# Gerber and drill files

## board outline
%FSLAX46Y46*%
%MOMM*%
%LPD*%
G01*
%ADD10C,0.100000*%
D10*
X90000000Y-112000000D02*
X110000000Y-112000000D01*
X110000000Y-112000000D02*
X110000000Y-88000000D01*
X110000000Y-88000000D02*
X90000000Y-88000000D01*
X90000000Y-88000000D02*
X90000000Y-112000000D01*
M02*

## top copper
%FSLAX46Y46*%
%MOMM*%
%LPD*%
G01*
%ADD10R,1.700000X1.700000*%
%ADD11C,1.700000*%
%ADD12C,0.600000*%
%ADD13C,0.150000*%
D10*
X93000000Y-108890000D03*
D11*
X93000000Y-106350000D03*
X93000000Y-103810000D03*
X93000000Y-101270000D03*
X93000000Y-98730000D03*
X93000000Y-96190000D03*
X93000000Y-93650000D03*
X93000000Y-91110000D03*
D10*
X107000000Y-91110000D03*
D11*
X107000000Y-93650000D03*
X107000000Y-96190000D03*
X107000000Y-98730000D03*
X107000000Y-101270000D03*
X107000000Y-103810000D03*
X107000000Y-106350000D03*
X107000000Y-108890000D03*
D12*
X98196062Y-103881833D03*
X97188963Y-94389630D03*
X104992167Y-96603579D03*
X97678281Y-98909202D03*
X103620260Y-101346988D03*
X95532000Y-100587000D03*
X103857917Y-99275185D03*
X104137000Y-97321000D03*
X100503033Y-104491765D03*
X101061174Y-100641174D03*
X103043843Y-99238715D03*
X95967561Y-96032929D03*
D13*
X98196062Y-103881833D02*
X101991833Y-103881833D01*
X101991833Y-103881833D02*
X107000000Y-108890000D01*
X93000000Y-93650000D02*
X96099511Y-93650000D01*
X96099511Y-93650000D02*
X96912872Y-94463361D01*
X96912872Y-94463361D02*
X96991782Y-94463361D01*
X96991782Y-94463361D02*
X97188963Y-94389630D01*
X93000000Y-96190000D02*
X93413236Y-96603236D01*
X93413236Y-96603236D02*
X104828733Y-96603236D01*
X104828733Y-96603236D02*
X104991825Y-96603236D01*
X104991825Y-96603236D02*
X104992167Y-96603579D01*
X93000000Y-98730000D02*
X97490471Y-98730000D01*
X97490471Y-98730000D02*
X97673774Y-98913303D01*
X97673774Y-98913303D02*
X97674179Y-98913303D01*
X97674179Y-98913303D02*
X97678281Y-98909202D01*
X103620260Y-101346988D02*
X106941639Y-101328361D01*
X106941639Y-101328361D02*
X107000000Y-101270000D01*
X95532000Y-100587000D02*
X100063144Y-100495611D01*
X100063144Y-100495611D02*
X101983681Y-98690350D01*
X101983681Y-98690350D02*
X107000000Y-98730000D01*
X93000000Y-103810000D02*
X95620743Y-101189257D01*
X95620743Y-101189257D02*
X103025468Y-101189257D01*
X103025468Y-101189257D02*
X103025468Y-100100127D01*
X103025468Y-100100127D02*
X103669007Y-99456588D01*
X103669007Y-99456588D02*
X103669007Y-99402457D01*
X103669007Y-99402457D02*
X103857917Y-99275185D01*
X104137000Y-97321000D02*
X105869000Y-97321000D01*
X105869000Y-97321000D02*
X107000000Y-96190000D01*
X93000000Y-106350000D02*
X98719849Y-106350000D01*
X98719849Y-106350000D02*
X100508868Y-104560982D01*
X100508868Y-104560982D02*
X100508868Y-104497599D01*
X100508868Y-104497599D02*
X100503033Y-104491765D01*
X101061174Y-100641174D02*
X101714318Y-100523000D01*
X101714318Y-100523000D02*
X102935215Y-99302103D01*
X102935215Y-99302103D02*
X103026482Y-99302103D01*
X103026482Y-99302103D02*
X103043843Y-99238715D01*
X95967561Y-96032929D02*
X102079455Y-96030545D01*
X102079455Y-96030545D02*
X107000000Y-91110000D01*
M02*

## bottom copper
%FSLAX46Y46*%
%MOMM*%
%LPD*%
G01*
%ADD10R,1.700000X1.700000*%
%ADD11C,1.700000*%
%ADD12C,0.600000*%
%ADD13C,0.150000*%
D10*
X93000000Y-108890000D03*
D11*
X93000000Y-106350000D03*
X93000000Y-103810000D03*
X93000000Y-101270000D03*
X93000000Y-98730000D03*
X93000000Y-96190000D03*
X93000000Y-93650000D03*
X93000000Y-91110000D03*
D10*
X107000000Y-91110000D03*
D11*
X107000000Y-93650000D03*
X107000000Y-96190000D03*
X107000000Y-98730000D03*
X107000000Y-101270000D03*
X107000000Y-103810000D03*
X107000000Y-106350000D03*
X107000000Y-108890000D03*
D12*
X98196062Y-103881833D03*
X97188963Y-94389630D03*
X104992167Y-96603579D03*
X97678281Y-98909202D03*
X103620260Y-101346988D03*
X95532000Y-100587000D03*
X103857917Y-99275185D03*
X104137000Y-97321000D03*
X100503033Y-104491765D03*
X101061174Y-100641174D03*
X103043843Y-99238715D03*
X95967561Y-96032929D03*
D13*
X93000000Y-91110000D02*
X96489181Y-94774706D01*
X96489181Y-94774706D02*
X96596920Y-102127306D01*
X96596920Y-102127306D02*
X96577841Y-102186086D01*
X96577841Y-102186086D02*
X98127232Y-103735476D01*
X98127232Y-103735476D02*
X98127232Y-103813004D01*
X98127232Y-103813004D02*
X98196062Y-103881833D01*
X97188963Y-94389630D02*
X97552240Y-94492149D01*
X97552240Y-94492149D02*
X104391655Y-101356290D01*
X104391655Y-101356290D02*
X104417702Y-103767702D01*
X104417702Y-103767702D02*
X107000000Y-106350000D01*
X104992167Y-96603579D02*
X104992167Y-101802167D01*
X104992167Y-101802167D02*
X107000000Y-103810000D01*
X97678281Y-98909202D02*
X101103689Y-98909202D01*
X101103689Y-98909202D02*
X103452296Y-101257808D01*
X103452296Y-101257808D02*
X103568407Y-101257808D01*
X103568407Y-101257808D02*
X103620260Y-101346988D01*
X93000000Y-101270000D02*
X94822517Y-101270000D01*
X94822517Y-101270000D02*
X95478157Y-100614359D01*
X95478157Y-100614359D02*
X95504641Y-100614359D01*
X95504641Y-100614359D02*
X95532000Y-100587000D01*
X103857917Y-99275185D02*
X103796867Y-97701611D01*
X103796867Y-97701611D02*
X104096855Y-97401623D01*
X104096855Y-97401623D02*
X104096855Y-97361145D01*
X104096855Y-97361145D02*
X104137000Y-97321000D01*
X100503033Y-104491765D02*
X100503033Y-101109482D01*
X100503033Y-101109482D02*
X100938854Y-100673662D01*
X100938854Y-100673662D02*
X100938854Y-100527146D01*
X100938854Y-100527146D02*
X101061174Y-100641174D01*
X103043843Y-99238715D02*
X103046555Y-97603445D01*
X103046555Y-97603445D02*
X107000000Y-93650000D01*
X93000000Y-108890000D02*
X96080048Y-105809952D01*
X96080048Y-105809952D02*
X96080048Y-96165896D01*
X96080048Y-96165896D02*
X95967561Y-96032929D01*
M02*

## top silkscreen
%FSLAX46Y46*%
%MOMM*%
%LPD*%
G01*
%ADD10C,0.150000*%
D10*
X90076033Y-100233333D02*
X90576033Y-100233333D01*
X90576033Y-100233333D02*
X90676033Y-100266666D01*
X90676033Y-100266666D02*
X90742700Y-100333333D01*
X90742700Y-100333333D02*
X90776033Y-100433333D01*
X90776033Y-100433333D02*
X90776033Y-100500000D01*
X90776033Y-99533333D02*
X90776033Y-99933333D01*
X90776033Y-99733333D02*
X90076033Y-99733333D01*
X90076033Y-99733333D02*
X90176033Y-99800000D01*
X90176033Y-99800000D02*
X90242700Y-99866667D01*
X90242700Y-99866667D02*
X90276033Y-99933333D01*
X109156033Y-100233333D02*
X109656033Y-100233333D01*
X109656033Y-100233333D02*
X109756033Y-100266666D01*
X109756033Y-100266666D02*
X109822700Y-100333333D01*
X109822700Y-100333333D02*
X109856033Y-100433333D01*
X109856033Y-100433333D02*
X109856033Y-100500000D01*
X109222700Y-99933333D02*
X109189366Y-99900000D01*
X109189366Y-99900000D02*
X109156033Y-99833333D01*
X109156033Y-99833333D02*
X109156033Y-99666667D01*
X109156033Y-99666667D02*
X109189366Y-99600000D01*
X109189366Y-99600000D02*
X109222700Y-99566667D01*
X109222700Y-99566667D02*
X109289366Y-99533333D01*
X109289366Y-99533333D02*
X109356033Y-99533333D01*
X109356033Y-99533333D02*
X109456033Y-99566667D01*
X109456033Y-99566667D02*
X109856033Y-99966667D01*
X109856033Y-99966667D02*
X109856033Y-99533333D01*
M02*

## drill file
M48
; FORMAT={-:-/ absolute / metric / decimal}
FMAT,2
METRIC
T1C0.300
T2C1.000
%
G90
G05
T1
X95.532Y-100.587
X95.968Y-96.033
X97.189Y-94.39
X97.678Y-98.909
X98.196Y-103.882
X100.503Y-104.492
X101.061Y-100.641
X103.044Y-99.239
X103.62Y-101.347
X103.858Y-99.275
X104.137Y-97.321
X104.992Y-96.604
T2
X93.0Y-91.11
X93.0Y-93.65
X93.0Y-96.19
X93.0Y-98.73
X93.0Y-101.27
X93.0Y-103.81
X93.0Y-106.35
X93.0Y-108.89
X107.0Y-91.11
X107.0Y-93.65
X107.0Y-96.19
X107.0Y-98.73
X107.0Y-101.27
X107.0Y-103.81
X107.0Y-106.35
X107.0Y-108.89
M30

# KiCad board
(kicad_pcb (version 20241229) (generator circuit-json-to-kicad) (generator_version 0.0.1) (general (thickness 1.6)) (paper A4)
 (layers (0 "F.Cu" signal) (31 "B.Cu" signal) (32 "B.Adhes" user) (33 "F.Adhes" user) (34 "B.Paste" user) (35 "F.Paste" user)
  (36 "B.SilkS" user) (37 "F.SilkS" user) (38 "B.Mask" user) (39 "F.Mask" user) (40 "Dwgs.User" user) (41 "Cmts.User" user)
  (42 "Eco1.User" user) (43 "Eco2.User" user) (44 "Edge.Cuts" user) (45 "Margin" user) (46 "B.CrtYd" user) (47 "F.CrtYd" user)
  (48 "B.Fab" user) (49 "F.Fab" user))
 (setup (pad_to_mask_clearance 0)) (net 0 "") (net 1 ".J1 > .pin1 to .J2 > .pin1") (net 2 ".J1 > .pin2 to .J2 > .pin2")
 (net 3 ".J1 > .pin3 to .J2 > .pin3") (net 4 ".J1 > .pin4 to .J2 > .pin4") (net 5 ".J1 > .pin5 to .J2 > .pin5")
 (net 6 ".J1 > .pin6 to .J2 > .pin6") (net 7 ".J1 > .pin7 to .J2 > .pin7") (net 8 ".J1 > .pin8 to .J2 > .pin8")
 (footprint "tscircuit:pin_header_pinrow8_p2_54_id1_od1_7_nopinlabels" (layer F.Cu) (at 93 100 90)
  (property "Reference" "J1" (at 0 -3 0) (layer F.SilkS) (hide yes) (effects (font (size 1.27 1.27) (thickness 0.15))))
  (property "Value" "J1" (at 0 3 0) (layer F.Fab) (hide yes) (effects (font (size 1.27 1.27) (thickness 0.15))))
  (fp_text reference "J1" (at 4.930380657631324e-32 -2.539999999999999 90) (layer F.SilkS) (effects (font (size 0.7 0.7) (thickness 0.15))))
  (pad "1" thru_hole rect (at -8.89 -3.4382291747912674e-16 90) (size 1.7 1.7) (drill 1) (layers *.Cu *.Mask)
   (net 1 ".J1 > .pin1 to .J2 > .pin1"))
  (pad "2" thru_hole circle (at -6.3500000000000005 3.8882535872928466e-16 0) (size 1.7 1.7) (drill 1) (layers *.Cu *.Mask)
   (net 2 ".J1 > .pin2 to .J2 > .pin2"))
  (pad "3" thru_hole circle (at -3.8100000000000005 2.332952152375708e-16 0) (size 1.7 1.7) (drill 1) (layers *.Cu *.Mask)
   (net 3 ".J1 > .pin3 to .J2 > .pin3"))
  (pad "4" thru_hole circle (at -1.2700000000000005 7.776507174585695e-17 0) (size 1.7 1.7) (drill 1) (layers *.Cu *.Mask)
   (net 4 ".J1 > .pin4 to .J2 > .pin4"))
  (pad "5" thru_hole circle (at 1.2699999999999996 -7.77650717458569e-17 0) (size 1.7 1.7) (drill 1) (layers *.Cu *.Mask)
   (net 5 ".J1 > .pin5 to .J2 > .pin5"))
  (pad "6" thru_hole circle (at 3.8099999999999987 -2.3329521523757073e-16 0) (size 1.7 1.7) (drill 1) (layers *.Cu *.Mask)
   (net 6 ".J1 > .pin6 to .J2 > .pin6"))
  (pad "7" thru_hole circle (at 6.35 -3.888253587292846e-16 0) (size 1.7 1.7) (drill 1) (layers *.Cu *.Mask)
   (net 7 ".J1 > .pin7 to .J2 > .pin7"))
  (pad "8" thru_hole circle (at 8.89 3.4382291747912674e-16 0) (size 1.7 1.7) (drill 1) (layers *.Cu *.Mask)
   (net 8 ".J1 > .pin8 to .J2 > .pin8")))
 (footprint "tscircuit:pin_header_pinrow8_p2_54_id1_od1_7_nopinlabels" (layer F.Cu) (at 107 100 270)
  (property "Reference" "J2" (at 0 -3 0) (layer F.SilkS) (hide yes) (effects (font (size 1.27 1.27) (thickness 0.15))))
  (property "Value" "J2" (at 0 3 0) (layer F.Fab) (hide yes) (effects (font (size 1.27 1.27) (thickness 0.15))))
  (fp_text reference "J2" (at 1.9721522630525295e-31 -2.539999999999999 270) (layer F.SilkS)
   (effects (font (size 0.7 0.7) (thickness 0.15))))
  (pad "1" thru_hole rect (at -8.89 -1.43290332737255e-16 270) (size 1.7 1.7) (drill 1) (layers *.Cu *.Mask)
   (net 1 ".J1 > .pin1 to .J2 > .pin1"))
  (pad "2" thru_hole circle (at -6.3500000000000005 2.782976564877288e-16 0) (size 1.7 1.7) (drill 1) (layers *.Cu *.Mask)
   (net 2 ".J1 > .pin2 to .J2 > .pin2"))
  (pad "3" thru_hole circle (at -3.8100000000000005 -1.8829277398741286e-16 0) (size 1.7 1.7) (drill 1) (layers *.Cu *.Mask)
   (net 3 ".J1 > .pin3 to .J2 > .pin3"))
  (pad "4" thru_hole circle (at -1.2700000000000005 2.3329521523757087e-16 0) (size 1.7 1.7) (drill 1) (layers *.Cu *.Mask)
   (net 4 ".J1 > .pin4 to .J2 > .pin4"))
  (pad "5" thru_hole circle (at 1.2699999999999996 -2.332952152375707e-16 0) (size 1.7 1.7) (drill 1) (layers *.Cu *.Mask)
   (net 5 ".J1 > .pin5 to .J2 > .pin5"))
  (pad "6" thru_hole circle (at 3.8099999999999987 1.8829277398741315e-16 0) (size 1.7 1.7) (drill 1) (layers *.Cu *.Mask)
   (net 6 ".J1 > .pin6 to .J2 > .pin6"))
  (pad "7" thru_hole circle (at 6.35 -2.782976564877286e-16 0) (size 1.7 1.7) (drill 1) (layers *.Cu *.Mask)
   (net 7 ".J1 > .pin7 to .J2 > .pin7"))
  (pad "8" thru_hole circle (at 8.89 1.43290332737255e-16 0) (size 1.7 1.7) (drill 1) (layers *.Cu *.Mask)
   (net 8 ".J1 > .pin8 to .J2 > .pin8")))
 (segment (start 93 91.11) (end 96.48918098719415 94.77470608881917) (width 0.15) (layer B.Cu) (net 8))
 (segment (start 96.48918098719415 94.77470608881917) (end 96.59692016415507 102.12730558444845) (width 0.15) (layer B.Cu) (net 8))
 (segment (start 96.59692016415507 102.12730558444845) (end 96.57784136417371 102.18608558049488) (width 0.15) (layer B.Cu) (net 8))
 (segment (start 96.57784136417371 102.18608558049488) (end 98.12723205798244 103.73547627430361) (width 0.15) (layer B.Cu) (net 8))
 (segment (start 98.12723205798244 103.73547627430361) (end 98.12723205798244 103.81300374321155) (width 0.15) (layer B.Cu) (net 8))
 (segment (start 98.12723205798244 103.81300374321155) (end 98.19606154724926 103.88183323247839) (width 0.15) (layer B.Cu) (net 8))
 (segment (start 98.19606154724926 103.88183323247839) (end 101.99183323247838 103.88183323247839) (width 0.15) (layer F.Cu) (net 8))
 (segment (start 101.99183323247838 103.88183323247839) (end 107 108.89) (width 0.15) (layer F.Cu) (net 8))
 (segment (start 93 93.65) (end 96.09951070501047 93.65) (width 0.15) (layer F.Cu) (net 7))
 (segment (start 96.09951070501047 93.65) (end 96.91287210251764 94.46336139750716) (width 0.15) (layer F.Cu) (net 7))
 (segment (start 96.91287210251764 94.46336139750716) (end 96.9917818220078 94.46336139750716) (width 0.15) (layer F.Cu) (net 7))
 (segment (start 96.9917818220078 94.46336139750716) (end 97.18896336907312 94.38963020554995) (width 0.15) (layer F.Cu) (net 7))
 (segment (start 97.18896336907312 94.38963020554995) (end 97.55224041660168 94.49214945666995) (width 0.15) (layer B.Cu) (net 7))
 (segment (start 97.55224041660168 94.49214945666995) (end 104.39165508828214 101.35628968946591) (width 0.15) (layer B.Cu) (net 7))
 (segment (start 104.39165508828214 101.35628968946591) (end 104.41770178162538 103.76770178162539) (width 0.15) (layer B.Cu) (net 7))
 (segment (start 104.41770178162538 103.76770178162539) (end 107 106.35) (width 0.15) (layer B.Cu) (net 7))
 (segment (start 93 96.19) (end 93.41323636103994 96.60323636103995) (width 0.15) (layer F.Cu) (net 6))
 (segment (start 93.41323636103994 96.60323636103995) (end 104.82873285592359 96.60323636103995) (width 0.15) (layer F.Cu) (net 6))
 (segment (start 104.82873285592359 96.60323636103995) (end 104.99182496950935 96.60323636103995) (width 0.15) (layer F.Cu) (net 6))
 (segment (start 104.99182496950935 96.60323636103995) (end 104.99216738752625 96.60357877905685) (width 0.15) (layer F.Cu) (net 6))
 (segment (start 104.99216738752625 96.60357877905685) (end 104.99216738752625 101.80216738752625) (width 0.15) (layer B.Cu) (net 6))
 (segment (start 104.99216738752625 101.80216738752625) (end 107 103.81) (width 0.15) (layer B.Cu) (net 6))
 (segment (start 93 98.73) (end 97.4904706501815 98.73) (width 0.15) (layer F.Cu) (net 5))
 (segment (start 97.4904706501815 98.73) (end 97.67377372562832 98.91330307544683) (width 0.15) (layer F.Cu) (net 5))
 (segment (start 97.67377372562832 98.91330307544683) (end 97.67417929996407 98.91330307544683) (width 0.15) (layer F.Cu) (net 5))
 (segment (start 97.67417929996407 98.91330307544683) (end 97.67828061547938 98.90920175993152) (width 0.15) (layer F.Cu) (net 5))
 (segment (start 97.67828061547938 98.90920175993152) (end 101.10368933616985 98.90920175993152) (width 0.15) (layer B.Cu) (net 5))
 (segment (start 101.10368933616985 98.90920175993152) (end 103.45229571378549 101.25780813754716) (width 0.15) (layer B.Cu) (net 5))
 (segment (start 103.45229571378549 101.25780813754716) (end 103.56840657012297 101.25780813754716) (width 0.15) (layer B.Cu) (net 5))
 (segment (start 103.56840657012297 101.25780813754716) (end 103.62026031462429 101.34698813464169) (width 0.15) (layer B.Cu) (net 5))
 (segment (start 103.62026031462429 101.34698813464169) (end 106.9416390042992 101.32836099570079) (width 0.15) (layer F.Cu) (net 5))
 (segment (start 106.9416390042992 101.32836099570079) (end 107 101.27) (width 0.15) (layer F.Cu) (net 5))
 (segment (start 93 101.27) (end 94.82251675877609 101.27) (width 0.15) (layer B.Cu) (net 4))
 (segment (start 94.82251675877609 101.27) (end 95.47815735352212 100.61435940525396) (width 0.15) (layer B.Cu) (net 4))
 (segment (start 95.47815735352212 100.61435940525396) (end 95.50464059474604 100.61435940525396) (width 0.15) (layer B.Cu) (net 4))
 (segment (start 95.50464059474604 100.61435940525396) (end 95.532 100.587) (width 0.15) (layer B.Cu) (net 4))
 (segment (start 95.532 100.587) (end 100.06314429543538 100.49561075931808) (width 0.15) (layer F.Cu) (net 4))
 (segment (start 100.06314429543538 100.49561075931808) (end 101.98368114263367 98.69034978552132) (width 0.15) (layer F.Cu) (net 4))
 (segment (start 101.98368114263367 98.69034978552132) (end 107 98.73) (width 0.15) (layer F.Cu) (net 4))
 (segment (start 93 103.81) (end 95.62074287706905 101.18925712293095) (width 0.15) (layer F.Cu) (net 3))
 (segment (start 95.62074287706905 101.18925712293095) (end 103.02546808352147 101.18925712293095) (width 0.15) (layer F.Cu) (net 3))
 (segment (start 103.02546808352147 101.18925712293095) (end 103.02546808352147 100.10012666166597) (width 0.15) (layer F.Cu) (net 3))
 (segment (start 103.02546808352147 100.10012666166597) (end 103.66900690522947 99.45658783995798) (width 0.15) (layer F.Cu) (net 3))
 (segment (start 103.66900690522947 99.45658783995798) (end 103.66900690522947 99.40245684582911) (width 0.15) (layer F.Cu) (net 3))
 (segment (start 103.66900690522947 99.40245684582911) (end 103.8579173105221 99.27518494102709) (width 0.15) (layer F.Cu) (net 3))
 (segment (start 103.8579173105221 99.27518494102709) (end 103.79686670851132 97.70161130617477) (width 0.15) (layer B.Cu) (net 3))
 (segment (start 103.79686670851132 97.70161130617477) (end 104.09685540270614 97.40162261197995) (width 0.15) (layer B.Cu) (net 3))
 (segment (start 104.09685540270614 97.40162261197995) (end 104.09685540270614 97.36114459729386) (width 0.15) (layer B.Cu) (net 3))
 (segment (start 104.09685540270614 97.36114459729386) (end 104.137 97.321) (width 0.15) (layer B.Cu) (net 3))
 (segment (start 104.137 97.321) (end 105.869 97.321) (width 0.15) (layer F.Cu) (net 3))
 (segment (start 105.869 97.321) (end 107 96.19) (width 0.15) (layer F.Cu) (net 3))
 (segment (start 93 106.35) (end 98.7198491619646 106.35) (width 0.15) (layer F.Cu) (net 2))
 (segment (start 98.7198491619646 106.35) (end 100.50886762465589 104.56098153730872) (width 0.15) (layer F.Cu) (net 2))
 (segment (start 100.50886762465589 104.56098153730872) (end 100.50886762465589 104.4975992692856) (width 0.15) (layer F.Cu) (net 2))
 (segment (start 100.50886762465589 104.4975992692856) (end 100.50303304048767 104.49176468511739) (width 0.15) (layer F.Cu) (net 2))
 (segment (start 100.50303304048767 104.49176468511739) (end 100.50303304048767 101.10948222442919) (width 0.15) (layer B.Cu) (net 2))
 (segment (start 100.50303304048767 101.10948222442919) (end 100.9388536453849 100.67366161953197) (width 0.15) (layer B.Cu) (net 2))
 (segment (start 100.9388536453849 100.67366161953197) (end 100.9388536453849 100.52714635461511) (width 0.15) (layer B.Cu) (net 2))
 (segment (start 100.9388536453849 100.52714635461511) (end 101.06117406788027 100.64117406788027) (width 0.15) (layer B.Cu) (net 2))
 (segment (start 101.06117406788027 100.64117406788027) (end 101.71431847201694 100.523) (width 0.15) (layer F.Cu) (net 2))
 (segment (start 101.71431847201694 100.523) (end 102.93521499482401 99.30210347719294) (width 0.15) (layer F.Cu) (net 2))
 (segment (start 102.93521499482401 99.30210347719294) (end 103.02648239623579 99.30210347719294) (width 0.15) (layer F.Cu) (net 2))
 (segment (start 103.02648239623579 99.30210347719294) (end 103.04384317916282 99.23871527461283) (width 0.15) (layer F.Cu) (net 2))
 (segment (start 103.04384317916282 99.23871527461283) (end 103.04655535055535 97.60344464944465) (width 0.15) (layer B.Cu) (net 2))
 (segment (start 103.04655535055535 97.60344464944465) (end 107 93.65) (width 0.15) (layer B.Cu) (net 2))
 (segment (start 93 108.89) (end 96.08004797280218 105.80995202719782) (width 0.15) (layer B.Cu) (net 1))
 (segment (start 96.08004797280218 105.80995202719782) (end 96.08004797280218 96.16589625905438) (width 0.15) (layer B.Cu) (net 1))
 (segment (start 96.08004797280218 96.16589625905438) (end 95.96756082225403 96.03292937672686) (width 0.15) (layer B.Cu) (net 1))
 (segment (start 95.96756082225403 96.03292937672686) (end 102.07945464537505 96.03054535462495) (width 0.15) (layer F.Cu) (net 1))
 (segment (start 102.07945464537505 96.03054535462495) (end 107 91.11) (width 0.15) (layer F.Cu) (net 1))
 (gr_line (start 90 112) (end 110 112) (width 0.1) (layer Edge.Cuts))
 (gr_line (start 110 112) (end 110 88) (width 0.1) (layer Edge.Cuts))
 (gr_line (start 110 88) (end 90 88) (width 0.1) (layer Edge.Cuts))
 (gr_line (start 90 88) (end 90 112) (width 0.1) (layer Edge.Cuts))
 (via (at 98.19606154724926 103.88183323247839) (size 0.6) (drill 0.3) (layers F.Cu B.Cu) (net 8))
 (via (at 97.18896336907312 94.38963020554995) (size 0.6) (drill 0.3) (layers F.Cu B.Cu) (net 7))
 (via (at 104.99216738752625 96.60357877905685) (size 0.6) (drill 0.3) (layers F.Cu B.Cu) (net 6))
 (via (at 97.67828061547938 98.90920175993152) (size 0.6) (drill 0.3) (layers F.Cu B.Cu) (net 5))
 (via (at 103.62026031462429 101.34698813464169) (size 0.6) (drill 0.3) (layers F.Cu B.Cu) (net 5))
 (via (at 95.532 100.587) (size 0.6) (drill 0.3) (layers F.Cu B.Cu) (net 4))
 (via (at 103.8579173105221 99.27518494102709) (size 0.6) (drill 0.3) (layers F.Cu B.Cu) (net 3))
 (via (at 104.137 97.321) (size 0.6) (drill 0.3) (layers F.Cu B.Cu) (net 3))
 (via (at 100.50303304048767 104.49176468511739) (size 0.6) (drill 0.3) (layers F.Cu B.Cu) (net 2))
 (via (at 101.06117406788027 100.64117406788027) (size 0.6) (drill 0.3) (layers F.Cu B.Cu) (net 2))
 (via (at 103.04384317916282 99.23871527461283) (size 0.6) (drill 0.3) (layers F.Cu B.Cu) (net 2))
 (via (at 95.96756082225403 96.03292937672686) (size 0.6) (drill 0.3) (layers F.Cu B.Cu) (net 1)))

